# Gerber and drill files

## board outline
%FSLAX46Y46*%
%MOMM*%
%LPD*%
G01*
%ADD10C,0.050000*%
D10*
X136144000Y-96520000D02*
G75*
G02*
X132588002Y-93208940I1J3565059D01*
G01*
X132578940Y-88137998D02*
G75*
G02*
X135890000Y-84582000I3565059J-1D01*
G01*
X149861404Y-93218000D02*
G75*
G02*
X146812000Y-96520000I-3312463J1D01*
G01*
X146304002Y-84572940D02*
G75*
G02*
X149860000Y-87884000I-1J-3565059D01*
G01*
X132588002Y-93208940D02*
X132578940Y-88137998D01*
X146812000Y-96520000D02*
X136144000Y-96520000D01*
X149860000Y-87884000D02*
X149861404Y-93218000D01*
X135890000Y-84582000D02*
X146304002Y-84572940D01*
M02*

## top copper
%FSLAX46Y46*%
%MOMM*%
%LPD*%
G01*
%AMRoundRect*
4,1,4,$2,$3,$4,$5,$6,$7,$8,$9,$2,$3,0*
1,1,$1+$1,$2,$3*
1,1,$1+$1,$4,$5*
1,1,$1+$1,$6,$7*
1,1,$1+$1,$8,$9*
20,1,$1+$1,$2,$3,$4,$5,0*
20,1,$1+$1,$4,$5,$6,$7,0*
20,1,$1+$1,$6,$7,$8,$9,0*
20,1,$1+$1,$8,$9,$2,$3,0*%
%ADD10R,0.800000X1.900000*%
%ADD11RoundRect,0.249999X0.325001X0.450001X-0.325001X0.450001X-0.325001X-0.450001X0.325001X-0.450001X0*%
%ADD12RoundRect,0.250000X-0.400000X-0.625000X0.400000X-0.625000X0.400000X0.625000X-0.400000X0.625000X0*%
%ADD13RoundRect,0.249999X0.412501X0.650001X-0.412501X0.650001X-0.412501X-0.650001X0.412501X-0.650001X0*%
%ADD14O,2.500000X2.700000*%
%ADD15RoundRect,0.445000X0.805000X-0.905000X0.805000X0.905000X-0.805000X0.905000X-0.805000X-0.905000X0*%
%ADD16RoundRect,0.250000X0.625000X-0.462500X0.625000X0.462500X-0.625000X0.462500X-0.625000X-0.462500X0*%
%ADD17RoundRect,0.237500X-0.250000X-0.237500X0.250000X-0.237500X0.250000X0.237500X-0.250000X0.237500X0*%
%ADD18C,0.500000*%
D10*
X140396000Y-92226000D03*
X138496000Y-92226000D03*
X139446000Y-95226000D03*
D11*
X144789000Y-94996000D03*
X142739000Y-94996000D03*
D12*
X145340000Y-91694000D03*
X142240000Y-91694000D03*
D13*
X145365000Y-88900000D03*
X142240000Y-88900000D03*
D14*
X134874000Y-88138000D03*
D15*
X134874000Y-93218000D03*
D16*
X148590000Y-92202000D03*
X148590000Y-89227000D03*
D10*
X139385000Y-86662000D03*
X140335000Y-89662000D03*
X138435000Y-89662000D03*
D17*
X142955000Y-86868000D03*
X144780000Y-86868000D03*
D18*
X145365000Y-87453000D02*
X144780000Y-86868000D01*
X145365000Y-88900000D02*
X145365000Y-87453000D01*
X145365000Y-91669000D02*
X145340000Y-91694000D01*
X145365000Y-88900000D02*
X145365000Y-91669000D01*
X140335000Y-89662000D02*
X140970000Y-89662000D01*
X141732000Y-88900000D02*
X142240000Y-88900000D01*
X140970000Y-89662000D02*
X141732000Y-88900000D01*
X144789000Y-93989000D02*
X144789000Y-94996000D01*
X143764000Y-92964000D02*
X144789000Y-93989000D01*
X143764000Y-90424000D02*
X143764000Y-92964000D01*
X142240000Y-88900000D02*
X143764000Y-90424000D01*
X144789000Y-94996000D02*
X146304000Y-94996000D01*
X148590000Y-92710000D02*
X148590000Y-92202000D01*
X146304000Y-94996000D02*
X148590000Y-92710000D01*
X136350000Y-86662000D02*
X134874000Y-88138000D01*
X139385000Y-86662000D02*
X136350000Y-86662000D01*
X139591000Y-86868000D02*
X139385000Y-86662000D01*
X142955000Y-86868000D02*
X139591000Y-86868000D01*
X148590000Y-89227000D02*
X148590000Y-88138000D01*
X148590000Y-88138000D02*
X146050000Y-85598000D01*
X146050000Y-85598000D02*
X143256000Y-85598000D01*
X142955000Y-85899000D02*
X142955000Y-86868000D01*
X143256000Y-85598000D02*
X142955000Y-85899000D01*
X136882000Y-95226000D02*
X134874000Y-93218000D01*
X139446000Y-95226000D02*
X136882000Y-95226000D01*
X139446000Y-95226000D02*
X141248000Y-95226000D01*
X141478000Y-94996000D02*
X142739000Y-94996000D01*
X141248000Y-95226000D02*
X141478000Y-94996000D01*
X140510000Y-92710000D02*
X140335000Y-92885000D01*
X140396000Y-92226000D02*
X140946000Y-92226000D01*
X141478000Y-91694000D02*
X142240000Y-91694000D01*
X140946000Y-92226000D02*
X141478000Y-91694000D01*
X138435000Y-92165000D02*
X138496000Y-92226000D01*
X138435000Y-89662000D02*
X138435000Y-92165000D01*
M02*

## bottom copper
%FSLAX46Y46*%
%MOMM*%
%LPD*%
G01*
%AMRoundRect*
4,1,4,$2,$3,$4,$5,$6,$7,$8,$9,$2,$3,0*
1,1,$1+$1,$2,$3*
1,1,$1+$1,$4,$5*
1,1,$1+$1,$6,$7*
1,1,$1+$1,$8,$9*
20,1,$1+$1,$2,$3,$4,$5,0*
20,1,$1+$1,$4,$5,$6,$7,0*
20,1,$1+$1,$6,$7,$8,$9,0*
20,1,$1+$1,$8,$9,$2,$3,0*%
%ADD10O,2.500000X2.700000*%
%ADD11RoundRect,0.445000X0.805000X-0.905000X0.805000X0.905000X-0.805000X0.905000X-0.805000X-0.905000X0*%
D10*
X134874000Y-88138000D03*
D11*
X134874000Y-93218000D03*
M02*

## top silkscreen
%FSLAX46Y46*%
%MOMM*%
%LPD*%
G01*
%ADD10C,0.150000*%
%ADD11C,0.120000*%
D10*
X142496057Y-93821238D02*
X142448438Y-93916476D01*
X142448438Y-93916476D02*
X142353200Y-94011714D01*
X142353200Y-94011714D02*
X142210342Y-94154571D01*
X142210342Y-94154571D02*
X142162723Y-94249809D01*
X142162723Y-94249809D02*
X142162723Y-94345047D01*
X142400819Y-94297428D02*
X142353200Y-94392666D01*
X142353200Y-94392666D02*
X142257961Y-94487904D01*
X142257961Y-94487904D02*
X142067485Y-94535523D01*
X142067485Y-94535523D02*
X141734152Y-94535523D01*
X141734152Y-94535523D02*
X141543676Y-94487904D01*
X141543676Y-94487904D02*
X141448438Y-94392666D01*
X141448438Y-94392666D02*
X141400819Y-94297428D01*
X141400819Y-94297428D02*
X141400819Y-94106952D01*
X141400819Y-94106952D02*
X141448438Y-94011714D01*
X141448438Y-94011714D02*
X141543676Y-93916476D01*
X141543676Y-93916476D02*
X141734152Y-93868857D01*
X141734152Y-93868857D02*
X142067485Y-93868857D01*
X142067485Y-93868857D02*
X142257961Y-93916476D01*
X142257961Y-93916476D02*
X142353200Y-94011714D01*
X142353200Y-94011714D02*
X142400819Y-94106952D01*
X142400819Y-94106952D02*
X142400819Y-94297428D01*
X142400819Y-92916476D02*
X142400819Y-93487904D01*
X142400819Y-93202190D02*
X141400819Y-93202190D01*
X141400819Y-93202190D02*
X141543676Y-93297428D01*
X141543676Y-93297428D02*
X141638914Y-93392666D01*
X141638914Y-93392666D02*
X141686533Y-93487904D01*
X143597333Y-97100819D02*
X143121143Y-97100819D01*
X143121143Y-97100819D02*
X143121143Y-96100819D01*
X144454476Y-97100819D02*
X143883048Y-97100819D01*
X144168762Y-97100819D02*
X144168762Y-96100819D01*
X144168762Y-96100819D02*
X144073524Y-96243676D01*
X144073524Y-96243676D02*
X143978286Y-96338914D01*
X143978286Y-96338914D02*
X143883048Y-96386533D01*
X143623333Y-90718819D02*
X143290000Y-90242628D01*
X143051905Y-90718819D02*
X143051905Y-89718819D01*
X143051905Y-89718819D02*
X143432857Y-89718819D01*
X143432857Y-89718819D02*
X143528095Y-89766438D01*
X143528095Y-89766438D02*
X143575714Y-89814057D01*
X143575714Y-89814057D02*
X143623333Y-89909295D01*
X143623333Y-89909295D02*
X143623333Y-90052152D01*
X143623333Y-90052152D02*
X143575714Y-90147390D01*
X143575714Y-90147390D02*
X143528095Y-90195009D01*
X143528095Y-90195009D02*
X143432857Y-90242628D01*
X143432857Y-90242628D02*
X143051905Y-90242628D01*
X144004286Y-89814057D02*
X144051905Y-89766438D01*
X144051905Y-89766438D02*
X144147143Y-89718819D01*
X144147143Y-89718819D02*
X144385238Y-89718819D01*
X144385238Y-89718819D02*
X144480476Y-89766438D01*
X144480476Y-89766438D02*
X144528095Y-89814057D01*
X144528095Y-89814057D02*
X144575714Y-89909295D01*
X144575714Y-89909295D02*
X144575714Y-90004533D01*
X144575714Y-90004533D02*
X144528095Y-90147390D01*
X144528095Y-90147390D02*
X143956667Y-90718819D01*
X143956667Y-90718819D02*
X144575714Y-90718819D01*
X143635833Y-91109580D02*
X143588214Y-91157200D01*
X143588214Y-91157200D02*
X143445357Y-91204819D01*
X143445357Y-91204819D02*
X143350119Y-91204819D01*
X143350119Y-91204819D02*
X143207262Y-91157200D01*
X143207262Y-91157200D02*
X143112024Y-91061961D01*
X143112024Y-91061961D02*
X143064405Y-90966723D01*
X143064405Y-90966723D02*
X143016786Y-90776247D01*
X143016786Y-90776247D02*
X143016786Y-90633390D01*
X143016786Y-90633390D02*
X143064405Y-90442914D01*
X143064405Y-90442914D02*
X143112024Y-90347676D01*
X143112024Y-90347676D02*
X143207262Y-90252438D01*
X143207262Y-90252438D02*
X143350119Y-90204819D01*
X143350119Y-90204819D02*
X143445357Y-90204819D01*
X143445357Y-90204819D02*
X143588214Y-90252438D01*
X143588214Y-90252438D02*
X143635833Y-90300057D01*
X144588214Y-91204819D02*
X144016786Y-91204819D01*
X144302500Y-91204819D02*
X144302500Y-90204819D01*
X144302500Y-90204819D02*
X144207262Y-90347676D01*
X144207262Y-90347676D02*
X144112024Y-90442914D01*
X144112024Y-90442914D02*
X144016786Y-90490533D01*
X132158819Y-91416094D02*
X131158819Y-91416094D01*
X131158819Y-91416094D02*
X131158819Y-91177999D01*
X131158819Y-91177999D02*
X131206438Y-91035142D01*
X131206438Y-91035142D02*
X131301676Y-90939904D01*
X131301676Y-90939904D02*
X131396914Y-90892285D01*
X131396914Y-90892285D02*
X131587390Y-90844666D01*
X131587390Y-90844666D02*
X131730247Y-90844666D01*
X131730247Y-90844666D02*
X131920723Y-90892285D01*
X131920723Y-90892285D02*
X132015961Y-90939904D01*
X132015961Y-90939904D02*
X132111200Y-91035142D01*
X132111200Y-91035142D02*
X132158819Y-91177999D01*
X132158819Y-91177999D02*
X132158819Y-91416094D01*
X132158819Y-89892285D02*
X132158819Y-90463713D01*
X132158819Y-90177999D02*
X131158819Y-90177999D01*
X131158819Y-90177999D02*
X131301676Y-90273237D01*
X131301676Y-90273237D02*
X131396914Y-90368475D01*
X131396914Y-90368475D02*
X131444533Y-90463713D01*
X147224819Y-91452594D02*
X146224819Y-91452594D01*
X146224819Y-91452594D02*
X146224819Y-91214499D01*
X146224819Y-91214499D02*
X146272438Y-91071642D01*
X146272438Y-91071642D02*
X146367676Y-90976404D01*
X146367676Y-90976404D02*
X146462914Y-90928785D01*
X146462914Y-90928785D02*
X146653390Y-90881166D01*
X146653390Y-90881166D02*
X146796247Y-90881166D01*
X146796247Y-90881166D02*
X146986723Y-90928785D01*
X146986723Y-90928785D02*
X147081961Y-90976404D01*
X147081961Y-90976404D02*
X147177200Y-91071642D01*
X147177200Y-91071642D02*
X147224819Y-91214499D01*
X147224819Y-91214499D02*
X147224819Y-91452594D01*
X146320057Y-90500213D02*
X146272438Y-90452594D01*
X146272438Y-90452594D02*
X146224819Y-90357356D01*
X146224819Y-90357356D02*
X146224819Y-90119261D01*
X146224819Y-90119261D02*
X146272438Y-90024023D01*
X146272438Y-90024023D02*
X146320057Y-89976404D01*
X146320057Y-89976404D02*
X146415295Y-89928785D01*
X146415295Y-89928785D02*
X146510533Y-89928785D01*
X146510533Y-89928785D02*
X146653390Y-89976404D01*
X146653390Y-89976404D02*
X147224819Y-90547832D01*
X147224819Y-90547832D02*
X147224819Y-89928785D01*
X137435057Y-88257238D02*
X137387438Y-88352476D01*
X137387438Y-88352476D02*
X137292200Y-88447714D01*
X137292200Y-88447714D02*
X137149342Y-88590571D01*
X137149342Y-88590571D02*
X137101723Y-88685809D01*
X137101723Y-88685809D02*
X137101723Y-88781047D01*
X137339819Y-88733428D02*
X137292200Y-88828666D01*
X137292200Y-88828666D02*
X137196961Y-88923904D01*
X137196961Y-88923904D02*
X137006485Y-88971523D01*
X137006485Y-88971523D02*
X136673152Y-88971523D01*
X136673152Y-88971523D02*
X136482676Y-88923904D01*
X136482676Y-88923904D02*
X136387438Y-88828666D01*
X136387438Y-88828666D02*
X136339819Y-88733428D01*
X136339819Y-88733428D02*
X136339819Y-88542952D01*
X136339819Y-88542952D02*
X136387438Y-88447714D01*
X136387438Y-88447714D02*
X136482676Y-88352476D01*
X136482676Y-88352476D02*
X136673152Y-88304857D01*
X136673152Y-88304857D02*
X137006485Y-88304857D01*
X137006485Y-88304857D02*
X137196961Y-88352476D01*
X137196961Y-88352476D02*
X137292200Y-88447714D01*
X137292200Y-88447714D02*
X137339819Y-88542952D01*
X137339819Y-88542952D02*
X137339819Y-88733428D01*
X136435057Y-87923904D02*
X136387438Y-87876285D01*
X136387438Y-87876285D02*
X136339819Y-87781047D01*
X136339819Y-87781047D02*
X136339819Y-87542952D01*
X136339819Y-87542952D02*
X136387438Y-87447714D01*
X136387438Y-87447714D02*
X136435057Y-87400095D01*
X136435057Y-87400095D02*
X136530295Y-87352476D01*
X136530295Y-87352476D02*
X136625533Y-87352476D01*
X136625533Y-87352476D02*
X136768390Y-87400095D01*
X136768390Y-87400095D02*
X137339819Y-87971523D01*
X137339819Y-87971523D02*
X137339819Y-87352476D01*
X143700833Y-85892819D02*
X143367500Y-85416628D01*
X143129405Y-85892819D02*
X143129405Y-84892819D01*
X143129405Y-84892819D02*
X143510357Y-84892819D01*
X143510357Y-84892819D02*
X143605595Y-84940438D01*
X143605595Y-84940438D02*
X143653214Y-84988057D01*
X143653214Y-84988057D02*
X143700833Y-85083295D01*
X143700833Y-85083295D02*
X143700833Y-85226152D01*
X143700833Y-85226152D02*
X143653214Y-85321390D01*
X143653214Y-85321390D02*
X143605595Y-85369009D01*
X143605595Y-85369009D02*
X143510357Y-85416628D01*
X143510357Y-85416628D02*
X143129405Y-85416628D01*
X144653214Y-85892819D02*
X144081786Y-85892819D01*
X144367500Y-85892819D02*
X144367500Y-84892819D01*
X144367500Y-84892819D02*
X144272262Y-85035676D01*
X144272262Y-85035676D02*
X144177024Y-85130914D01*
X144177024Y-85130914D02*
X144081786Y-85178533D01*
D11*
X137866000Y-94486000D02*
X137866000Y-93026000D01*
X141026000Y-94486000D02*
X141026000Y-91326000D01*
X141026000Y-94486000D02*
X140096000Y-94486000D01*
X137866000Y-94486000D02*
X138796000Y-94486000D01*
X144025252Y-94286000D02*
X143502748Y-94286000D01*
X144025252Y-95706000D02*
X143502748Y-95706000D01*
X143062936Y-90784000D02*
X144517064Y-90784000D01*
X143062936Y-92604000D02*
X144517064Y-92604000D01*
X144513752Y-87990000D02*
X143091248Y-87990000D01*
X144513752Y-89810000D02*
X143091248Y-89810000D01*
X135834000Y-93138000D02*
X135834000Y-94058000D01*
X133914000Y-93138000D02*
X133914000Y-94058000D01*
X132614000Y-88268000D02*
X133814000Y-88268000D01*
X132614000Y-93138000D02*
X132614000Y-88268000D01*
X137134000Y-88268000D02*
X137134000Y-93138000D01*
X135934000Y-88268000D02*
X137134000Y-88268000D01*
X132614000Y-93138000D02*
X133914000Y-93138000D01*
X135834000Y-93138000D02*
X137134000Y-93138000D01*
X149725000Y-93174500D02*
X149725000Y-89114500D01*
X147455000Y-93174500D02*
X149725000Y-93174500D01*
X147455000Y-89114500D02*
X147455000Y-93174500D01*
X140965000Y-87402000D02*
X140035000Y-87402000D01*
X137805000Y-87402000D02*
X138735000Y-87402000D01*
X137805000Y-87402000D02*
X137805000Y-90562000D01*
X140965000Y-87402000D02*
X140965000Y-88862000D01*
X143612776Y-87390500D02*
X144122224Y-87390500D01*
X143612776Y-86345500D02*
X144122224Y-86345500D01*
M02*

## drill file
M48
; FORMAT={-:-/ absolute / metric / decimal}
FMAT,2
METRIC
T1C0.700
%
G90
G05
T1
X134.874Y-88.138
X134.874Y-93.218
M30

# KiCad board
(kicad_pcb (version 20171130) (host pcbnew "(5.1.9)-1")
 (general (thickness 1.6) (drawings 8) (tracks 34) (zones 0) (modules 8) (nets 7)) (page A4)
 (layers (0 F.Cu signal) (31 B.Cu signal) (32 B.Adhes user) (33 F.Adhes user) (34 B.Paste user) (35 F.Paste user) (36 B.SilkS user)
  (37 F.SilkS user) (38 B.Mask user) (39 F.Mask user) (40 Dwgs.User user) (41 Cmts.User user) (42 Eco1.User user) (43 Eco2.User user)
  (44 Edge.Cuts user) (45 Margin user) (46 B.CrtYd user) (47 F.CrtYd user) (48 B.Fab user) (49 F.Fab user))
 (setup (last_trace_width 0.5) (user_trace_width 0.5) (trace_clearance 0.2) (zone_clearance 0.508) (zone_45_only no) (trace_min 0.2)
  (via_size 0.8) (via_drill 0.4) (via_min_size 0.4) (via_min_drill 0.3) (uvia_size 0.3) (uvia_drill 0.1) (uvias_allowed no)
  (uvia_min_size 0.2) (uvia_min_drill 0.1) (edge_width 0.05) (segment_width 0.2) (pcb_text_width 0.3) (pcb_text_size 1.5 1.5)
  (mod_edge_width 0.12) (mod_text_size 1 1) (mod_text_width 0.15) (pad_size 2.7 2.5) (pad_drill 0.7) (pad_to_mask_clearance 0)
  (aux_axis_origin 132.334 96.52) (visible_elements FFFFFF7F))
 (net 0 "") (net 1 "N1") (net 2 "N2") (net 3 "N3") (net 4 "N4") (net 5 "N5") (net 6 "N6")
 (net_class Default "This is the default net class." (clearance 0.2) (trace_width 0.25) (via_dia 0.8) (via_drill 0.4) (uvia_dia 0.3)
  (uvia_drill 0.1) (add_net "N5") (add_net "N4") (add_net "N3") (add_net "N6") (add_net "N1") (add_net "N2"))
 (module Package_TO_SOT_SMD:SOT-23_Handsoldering (layer F.Cu) (at 139.446 93.726 270)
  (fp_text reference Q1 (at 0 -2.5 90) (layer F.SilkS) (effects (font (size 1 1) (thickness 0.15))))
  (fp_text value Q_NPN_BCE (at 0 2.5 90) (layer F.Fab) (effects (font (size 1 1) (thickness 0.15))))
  (fp_line (start 0.76 1.58) (end -0.7 1.58) (layer F.SilkS) (width 0.12))
  (fp_line (start 0.76 -1.58) (end -2.4 -1.58) (layer F.SilkS) (width 0.12))
  (fp_line (start 0.76 -1.58) (end 0.76 -0.65) (layer F.SilkS) (width 0.12))
  (fp_line (start 0.76 1.58) (end 0.76 0.65) (layer F.SilkS) (width 0.12))
  (pad 1 smd rect (at -1.5 -0.95 270) (size 1.9 0.8) (layers F.Cu F.Paste F.Mask) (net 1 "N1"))
  (pad 2 smd rect (at -1.5 0.95 270) (size 1.9 0.8) (layers F.Cu F.Paste F.Mask) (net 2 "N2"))
  (pad 3 smd rect (at 1.5 0 270) (size 1.9 0.8) (layers F.Cu F.Paste F.Mask) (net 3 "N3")))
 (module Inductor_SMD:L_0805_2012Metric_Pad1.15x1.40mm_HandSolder (layer F.Cu) (at 143.764 94.996 180)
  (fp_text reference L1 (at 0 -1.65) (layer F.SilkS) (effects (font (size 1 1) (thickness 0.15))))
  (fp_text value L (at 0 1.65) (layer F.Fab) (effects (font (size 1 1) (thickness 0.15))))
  (fp_line (start -0.261252 0.71) (end 0.261252 0.71) (layer F.SilkS) (width 0.12))
  (fp_line (start -0.261252 -0.71) (end 0.261252 -0.71) (layer F.SilkS) (width 0.12))
  (pad 1 smd roundrect (at -1.025 0 180) (size 1.15 1.4) (layers F.Cu F.Paste F.Mask) (roundrect_rratio 0.2173904347826087) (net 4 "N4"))
  (pad 2 smd roundrect (at 1.025 0 180) (size 1.15 1.4) (layers F.Cu F.Paste F.Mask) (roundrect_rratio 0.2173904347826087) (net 3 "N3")))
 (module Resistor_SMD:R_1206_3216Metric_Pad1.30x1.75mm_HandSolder (layer F.Cu) (at 143.79 91.694)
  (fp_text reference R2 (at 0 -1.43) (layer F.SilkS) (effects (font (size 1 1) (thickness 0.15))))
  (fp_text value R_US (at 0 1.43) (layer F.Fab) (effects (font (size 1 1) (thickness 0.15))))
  (fp_line (start -0.727064 -0.91) (end 0.727064 -0.91) (layer F.SilkS) (width 0.12))
  (fp_line (start -0.727064 0.91) (end 0.727064 0.91) (layer F.SilkS) (width 0.12))
  (pad 2 smd roundrect (at 1.55 0) (size 1.3 1.75) (layers F.Cu F.Paste F.Mask) (roundrect_rratio 0.1923076923076923) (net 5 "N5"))
  (pad 1 smd roundrect (at -1.55 0) (size 1.3 1.75) (layers F.Cu F.Paste F.Mask) (roundrect_rratio 0.1923076923076923) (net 1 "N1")))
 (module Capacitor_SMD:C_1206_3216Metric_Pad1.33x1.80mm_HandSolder (layer F.Cu) (at 143.8025 88.9 180)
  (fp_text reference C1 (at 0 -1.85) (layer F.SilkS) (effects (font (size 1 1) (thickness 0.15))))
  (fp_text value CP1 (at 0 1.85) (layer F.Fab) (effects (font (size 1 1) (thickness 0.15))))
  (fp_line (start -0.711252 0.91) (end 0.711252 0.91) (layer F.SilkS) (width 0.12))
  (fp_line (start -0.711252 -0.91) (end 0.711252 -0.91) (layer F.SilkS) (width 0.12))
  (pad 1 smd roundrect (at -1.5625 0 180) (size 1.325 1.8) (layers F.Cu F.Paste F.Mask) (roundrect_rratio 0.1886784905660377) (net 5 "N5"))
  (pad 2 smd roundrect (at 1.5625 0 180) (size 1.325 1.8) (layers F.Cu F.Paste F.Mask) (roundrect_rratio 0.1886784905660377) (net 4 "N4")))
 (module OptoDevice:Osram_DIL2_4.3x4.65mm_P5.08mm (layer F.Cu) (at 134.874 93.218 90)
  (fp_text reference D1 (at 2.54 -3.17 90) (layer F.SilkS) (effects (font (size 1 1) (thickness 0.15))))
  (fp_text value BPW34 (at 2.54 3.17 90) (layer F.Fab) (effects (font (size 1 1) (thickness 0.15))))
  (fp_line (start 0.08 0.96) (end -0.84 0.96) (layer F.SilkS) (width 0.12))
  (fp_line (start 0.08 -0.96) (end -0.84 -0.96) (layer F.SilkS) (width 0.12))
  (fp_line (start 4.95 -2.26) (end 4.95 -1.06) (layer F.SilkS) (width 0.12))
  (fp_line (start 0.08 -2.26) (end 4.95 -2.26) (layer F.SilkS) (width 0.12))
  (fp_line (start 4.95 2.26) (end 0.08 2.26) (layer F.SilkS) (width 0.12))
  (fp_line (start 4.95 1.06) (end 4.95 2.26) (layer F.SilkS) (width 0.12))
  (fp_line (start 0.08 -2.26) (end 0.08 -0.96) (layer F.SilkS) (width 0.12))
  (fp_line (start 0.08 0.96) (end 0.08 2.26) (layer F.SilkS) (width 0.12))
  (pad 2 thru_hole oval (at 5.08 0 90) (size 2.7 2.5) (drill 0.7) (layers *.Cu *.Mask) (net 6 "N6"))
  (pad 1 thru_hole roundrect (at 0 0 90) (size 2.7 2.5) (drill 0.7) (layers *.Cu *.Mask) (roundrect_rratio 0.178) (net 3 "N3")))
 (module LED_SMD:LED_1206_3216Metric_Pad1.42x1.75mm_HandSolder (layer F.Cu) (at 148.59 90.7145 90)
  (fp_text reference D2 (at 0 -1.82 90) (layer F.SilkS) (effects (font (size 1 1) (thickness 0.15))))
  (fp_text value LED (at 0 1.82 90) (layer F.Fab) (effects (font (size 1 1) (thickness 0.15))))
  (fp_line (start -2.46 1.135) (end 1.6 1.135) (layer F.SilkS) (width 0.12))
  (fp_line (start -2.46 -1.135) (end -2.46 1.135) (layer F.SilkS) (width 0.12))
  (fp_line (start 1.6 -1.135) (end -2.46 -1.135) (layer F.SilkS) (width 0.12))
  (pad 1 smd roundrect (at -1.4875 0 90) (size 1.425 1.75) (layers F.Cu F.Paste F.Mask) (roundrect_rratio 0.1754385964912281) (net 4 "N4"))
  (pad 2 smd roundrect (at 1.4875 0 90) (size 1.425 1.75) (layers F.Cu F.Paste F.Mask) (roundrect_rratio 0.1754385964912281) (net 6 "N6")))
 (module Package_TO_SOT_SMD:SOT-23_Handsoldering (layer F.Cu) (at 139.385 88.162 90)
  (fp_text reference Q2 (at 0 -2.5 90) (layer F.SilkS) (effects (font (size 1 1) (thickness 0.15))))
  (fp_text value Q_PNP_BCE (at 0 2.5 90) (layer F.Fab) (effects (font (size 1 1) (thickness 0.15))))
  (fp_line (start 0.76 1.58) (end 0.76 0.65) (layer F.SilkS) (width 0.12))
  (fp_line (start 0.76 -1.58) (end 0.76 -0.65) (layer F.SilkS) (width 0.12))
  (fp_line (start 0.76 -1.58) (end -2.4 -1.58) (layer F.SilkS) (width 0.12))
  (fp_line (start 0.76 1.58) (end -0.7 1.58) (layer F.SilkS) (width 0.12))
  (pad 3 smd rect (at 1.5 0 90) (size 1.9 0.8) (layers F.Cu F.Paste F.Mask) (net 6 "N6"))
  (pad 2 smd rect (at -1.5 0.95 90) (size 1.9 0.8) (layers F.Cu F.Paste F.Mask) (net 4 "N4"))
  (pad 1 smd rect (at -1.5 -0.95 90) (size 1.9 0.8) (layers F.Cu F.Paste F.Mask) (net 2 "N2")))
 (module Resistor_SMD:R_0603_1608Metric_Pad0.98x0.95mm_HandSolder (layer F.Cu) (at 143.8675 86.868)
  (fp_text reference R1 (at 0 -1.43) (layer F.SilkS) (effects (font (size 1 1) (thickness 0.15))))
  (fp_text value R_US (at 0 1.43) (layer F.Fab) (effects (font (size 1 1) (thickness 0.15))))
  (fp_line (start -0.254724 0.5225) (end 0.254724 0.5225) (layer F.SilkS) (width 0.12))
  (fp_line (start -0.254724 -0.5225) (end 0.254724 -0.5225) (layer F.SilkS) (width 0.12))
  (pad 1 smd roundrect (at -0.9125 0) (size 0.975 0.95) (layers F.Cu F.Paste F.Mask) (roundrect_rratio 0.25) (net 6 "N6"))
  (pad 2 smd roundrect (at 0.9125 0) (size 0.975 0.95) (layers F.Cu F.Paste F.Mask) (roundrect_rratio 0.25) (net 5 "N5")))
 (gr_arc (start 136.144001 92.954941) (end 132.588002 93.20894) (angle -85.91438322) (layer Edge.Cuts) (width 0.05))
 (gr_arc (start 136.143999 88.137999) (end 135.89 84.582) (angle -85.91438322) (layer Edge.Cuts) (width 0.05))
 (gr_arc (start 146.548941 93.217999) (end 146.812 96.52) (angle -85.44504621) (layer Edge.Cuts) (width 0.05))
 (gr_arc (start 146.304001 88.137999) (end 149.86 87.884) (angle -85.91438203) (layer Edge.Cuts) (width 0.05))
 (gr_line (start 132.588002 93.20894) (end 132.57894 88.137998) (layer Edge.Cuts) (width 0.05))
 (gr_line (start 146.812 96.52) (end 136.144 96.52) (layer Edge.Cuts) (width 0.05))
 (gr_line (start 149.86 87.884) (end 149.861404 93.218) (layer Edge.Cuts) (width 0.05))
 (gr_line (start 135.89 84.582) (end 146.304002 84.57294) (layer Edge.Cuts) (width 0.05))
 (segment (start 145.365 87.453) (end 144.78 86.868) (width 0.5) (layer F.Cu) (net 5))
 (segment (start 145.365 88.9) (end 145.365 87.453) (width 0.5) (layer F.Cu) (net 5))
 (segment (start 145.365 91.669) (end 145.34 91.694) (width 0.5) (layer F.Cu) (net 5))
 (segment (start 145.365 88.9) (end 145.365 91.669) (width 0.5) (layer F.Cu) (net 5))
 (segment (start 140.335 89.662) (end 140.97 89.662) (width 0.5) (layer F.Cu) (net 4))
 (segment (start 141.732 88.9) (end 142.24 88.9) (width 0.5) (layer F.Cu) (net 4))
 (segment (start 140.97 89.662) (end 141.732 88.9) (width 0.5) (layer F.Cu) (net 4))
 (segment (start 144.789 93.989) (end 144.789 94.996) (width 0.5) (layer F.Cu) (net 4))
 (segment (start 143.764 92.964) (end 144.789 93.989) (width 0.5) (layer F.Cu) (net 4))
 (segment (start 143.764 90.424) (end 143.764 92.964) (width 0.5) (layer F.Cu) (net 4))
 (segment (start 142.24 88.9) (end 143.764 90.424) (width 0.5) (layer F.Cu) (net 4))
 (segment (start 144.789 94.996) (end 146.304 94.996) (width 0.5) (layer F.Cu) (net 4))
 (segment (start 148.59 92.71) (end 148.59 92.202) (width 0.5) (layer F.Cu) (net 4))
 (segment (start 146.304 94.996) (end 148.59 92.71) (width 0.5) (layer F.Cu) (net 4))
 (segment (start 136.35 86.662) (end 134.874 88.138) (width 0.5) (layer F.Cu) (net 6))
 (segment (start 139.385 86.662) (end 136.35 86.662) (width 0.5) (layer F.Cu) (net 6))
 (segment (start 139.591 86.868) (end 139.385 86.662) (width 0.5) (layer F.Cu) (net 6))
 (segment (start 142.955 86.868) (end 139.591 86.868) (width 0.5) (layer F.Cu) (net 6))
 (segment (start 148.59 89.227) (end 148.59 88.138) (width 0.5) (layer F.Cu) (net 6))
 (segment (start 148.59 88.138) (end 146.05 85.598) (width 0.5) (layer F.Cu) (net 6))
 (segment (start 146.05 85.598) (end 143.256 85.598) (width 0.5) (layer F.Cu) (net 6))
 (segment (start 142.955 85.899) (end 142.955 86.868) (width 0.5) (layer F.Cu) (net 6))
 (segment (start 143.256 85.598) (end 142.955 85.899) (width 0.5) (layer F.Cu) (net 6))
 (segment (start 136.882 95.226) (end 134.874 93.218) (width 0.5) (layer F.Cu) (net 3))
 (segment (start 139.446 95.226) (end 136.882 95.226) (width 0.5) (layer F.Cu) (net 3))
 (segment (start 139.446 95.226) (end 141.248 95.226) (width 0.5) (layer F.Cu) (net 3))
 (segment (start 141.478 94.996) (end 142.739 94.996) (width 0.5) (layer F.Cu) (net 3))
 (segment (start 141.248 95.226) (end 141.478 94.996) (width 0.5) (layer F.Cu) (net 3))
 (segment (start 140.51 92.71) (end 140.335 92.885) (width 0.5) (layer F.Cu) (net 1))
 (segment (start 140.396 92.226) (end 140.946 92.226) (width 0.5) (layer F.Cu) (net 1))
 (segment (start 141.478 91.694) (end 142.24 91.694) (width 0.5) (layer F.Cu) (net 1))
 (segment (start 140.946 92.226) (end 141.478 91.694) (width 0.5) (layer F.Cu) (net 1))
 (segment (start 138.435 92.165) (end 138.496 92.226) (width 0.5) (layer F.Cu) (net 2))
 (segment (start 138.435 89.662) (end 138.435 92.165) (width 0.5) (layer F.Cu) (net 2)))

